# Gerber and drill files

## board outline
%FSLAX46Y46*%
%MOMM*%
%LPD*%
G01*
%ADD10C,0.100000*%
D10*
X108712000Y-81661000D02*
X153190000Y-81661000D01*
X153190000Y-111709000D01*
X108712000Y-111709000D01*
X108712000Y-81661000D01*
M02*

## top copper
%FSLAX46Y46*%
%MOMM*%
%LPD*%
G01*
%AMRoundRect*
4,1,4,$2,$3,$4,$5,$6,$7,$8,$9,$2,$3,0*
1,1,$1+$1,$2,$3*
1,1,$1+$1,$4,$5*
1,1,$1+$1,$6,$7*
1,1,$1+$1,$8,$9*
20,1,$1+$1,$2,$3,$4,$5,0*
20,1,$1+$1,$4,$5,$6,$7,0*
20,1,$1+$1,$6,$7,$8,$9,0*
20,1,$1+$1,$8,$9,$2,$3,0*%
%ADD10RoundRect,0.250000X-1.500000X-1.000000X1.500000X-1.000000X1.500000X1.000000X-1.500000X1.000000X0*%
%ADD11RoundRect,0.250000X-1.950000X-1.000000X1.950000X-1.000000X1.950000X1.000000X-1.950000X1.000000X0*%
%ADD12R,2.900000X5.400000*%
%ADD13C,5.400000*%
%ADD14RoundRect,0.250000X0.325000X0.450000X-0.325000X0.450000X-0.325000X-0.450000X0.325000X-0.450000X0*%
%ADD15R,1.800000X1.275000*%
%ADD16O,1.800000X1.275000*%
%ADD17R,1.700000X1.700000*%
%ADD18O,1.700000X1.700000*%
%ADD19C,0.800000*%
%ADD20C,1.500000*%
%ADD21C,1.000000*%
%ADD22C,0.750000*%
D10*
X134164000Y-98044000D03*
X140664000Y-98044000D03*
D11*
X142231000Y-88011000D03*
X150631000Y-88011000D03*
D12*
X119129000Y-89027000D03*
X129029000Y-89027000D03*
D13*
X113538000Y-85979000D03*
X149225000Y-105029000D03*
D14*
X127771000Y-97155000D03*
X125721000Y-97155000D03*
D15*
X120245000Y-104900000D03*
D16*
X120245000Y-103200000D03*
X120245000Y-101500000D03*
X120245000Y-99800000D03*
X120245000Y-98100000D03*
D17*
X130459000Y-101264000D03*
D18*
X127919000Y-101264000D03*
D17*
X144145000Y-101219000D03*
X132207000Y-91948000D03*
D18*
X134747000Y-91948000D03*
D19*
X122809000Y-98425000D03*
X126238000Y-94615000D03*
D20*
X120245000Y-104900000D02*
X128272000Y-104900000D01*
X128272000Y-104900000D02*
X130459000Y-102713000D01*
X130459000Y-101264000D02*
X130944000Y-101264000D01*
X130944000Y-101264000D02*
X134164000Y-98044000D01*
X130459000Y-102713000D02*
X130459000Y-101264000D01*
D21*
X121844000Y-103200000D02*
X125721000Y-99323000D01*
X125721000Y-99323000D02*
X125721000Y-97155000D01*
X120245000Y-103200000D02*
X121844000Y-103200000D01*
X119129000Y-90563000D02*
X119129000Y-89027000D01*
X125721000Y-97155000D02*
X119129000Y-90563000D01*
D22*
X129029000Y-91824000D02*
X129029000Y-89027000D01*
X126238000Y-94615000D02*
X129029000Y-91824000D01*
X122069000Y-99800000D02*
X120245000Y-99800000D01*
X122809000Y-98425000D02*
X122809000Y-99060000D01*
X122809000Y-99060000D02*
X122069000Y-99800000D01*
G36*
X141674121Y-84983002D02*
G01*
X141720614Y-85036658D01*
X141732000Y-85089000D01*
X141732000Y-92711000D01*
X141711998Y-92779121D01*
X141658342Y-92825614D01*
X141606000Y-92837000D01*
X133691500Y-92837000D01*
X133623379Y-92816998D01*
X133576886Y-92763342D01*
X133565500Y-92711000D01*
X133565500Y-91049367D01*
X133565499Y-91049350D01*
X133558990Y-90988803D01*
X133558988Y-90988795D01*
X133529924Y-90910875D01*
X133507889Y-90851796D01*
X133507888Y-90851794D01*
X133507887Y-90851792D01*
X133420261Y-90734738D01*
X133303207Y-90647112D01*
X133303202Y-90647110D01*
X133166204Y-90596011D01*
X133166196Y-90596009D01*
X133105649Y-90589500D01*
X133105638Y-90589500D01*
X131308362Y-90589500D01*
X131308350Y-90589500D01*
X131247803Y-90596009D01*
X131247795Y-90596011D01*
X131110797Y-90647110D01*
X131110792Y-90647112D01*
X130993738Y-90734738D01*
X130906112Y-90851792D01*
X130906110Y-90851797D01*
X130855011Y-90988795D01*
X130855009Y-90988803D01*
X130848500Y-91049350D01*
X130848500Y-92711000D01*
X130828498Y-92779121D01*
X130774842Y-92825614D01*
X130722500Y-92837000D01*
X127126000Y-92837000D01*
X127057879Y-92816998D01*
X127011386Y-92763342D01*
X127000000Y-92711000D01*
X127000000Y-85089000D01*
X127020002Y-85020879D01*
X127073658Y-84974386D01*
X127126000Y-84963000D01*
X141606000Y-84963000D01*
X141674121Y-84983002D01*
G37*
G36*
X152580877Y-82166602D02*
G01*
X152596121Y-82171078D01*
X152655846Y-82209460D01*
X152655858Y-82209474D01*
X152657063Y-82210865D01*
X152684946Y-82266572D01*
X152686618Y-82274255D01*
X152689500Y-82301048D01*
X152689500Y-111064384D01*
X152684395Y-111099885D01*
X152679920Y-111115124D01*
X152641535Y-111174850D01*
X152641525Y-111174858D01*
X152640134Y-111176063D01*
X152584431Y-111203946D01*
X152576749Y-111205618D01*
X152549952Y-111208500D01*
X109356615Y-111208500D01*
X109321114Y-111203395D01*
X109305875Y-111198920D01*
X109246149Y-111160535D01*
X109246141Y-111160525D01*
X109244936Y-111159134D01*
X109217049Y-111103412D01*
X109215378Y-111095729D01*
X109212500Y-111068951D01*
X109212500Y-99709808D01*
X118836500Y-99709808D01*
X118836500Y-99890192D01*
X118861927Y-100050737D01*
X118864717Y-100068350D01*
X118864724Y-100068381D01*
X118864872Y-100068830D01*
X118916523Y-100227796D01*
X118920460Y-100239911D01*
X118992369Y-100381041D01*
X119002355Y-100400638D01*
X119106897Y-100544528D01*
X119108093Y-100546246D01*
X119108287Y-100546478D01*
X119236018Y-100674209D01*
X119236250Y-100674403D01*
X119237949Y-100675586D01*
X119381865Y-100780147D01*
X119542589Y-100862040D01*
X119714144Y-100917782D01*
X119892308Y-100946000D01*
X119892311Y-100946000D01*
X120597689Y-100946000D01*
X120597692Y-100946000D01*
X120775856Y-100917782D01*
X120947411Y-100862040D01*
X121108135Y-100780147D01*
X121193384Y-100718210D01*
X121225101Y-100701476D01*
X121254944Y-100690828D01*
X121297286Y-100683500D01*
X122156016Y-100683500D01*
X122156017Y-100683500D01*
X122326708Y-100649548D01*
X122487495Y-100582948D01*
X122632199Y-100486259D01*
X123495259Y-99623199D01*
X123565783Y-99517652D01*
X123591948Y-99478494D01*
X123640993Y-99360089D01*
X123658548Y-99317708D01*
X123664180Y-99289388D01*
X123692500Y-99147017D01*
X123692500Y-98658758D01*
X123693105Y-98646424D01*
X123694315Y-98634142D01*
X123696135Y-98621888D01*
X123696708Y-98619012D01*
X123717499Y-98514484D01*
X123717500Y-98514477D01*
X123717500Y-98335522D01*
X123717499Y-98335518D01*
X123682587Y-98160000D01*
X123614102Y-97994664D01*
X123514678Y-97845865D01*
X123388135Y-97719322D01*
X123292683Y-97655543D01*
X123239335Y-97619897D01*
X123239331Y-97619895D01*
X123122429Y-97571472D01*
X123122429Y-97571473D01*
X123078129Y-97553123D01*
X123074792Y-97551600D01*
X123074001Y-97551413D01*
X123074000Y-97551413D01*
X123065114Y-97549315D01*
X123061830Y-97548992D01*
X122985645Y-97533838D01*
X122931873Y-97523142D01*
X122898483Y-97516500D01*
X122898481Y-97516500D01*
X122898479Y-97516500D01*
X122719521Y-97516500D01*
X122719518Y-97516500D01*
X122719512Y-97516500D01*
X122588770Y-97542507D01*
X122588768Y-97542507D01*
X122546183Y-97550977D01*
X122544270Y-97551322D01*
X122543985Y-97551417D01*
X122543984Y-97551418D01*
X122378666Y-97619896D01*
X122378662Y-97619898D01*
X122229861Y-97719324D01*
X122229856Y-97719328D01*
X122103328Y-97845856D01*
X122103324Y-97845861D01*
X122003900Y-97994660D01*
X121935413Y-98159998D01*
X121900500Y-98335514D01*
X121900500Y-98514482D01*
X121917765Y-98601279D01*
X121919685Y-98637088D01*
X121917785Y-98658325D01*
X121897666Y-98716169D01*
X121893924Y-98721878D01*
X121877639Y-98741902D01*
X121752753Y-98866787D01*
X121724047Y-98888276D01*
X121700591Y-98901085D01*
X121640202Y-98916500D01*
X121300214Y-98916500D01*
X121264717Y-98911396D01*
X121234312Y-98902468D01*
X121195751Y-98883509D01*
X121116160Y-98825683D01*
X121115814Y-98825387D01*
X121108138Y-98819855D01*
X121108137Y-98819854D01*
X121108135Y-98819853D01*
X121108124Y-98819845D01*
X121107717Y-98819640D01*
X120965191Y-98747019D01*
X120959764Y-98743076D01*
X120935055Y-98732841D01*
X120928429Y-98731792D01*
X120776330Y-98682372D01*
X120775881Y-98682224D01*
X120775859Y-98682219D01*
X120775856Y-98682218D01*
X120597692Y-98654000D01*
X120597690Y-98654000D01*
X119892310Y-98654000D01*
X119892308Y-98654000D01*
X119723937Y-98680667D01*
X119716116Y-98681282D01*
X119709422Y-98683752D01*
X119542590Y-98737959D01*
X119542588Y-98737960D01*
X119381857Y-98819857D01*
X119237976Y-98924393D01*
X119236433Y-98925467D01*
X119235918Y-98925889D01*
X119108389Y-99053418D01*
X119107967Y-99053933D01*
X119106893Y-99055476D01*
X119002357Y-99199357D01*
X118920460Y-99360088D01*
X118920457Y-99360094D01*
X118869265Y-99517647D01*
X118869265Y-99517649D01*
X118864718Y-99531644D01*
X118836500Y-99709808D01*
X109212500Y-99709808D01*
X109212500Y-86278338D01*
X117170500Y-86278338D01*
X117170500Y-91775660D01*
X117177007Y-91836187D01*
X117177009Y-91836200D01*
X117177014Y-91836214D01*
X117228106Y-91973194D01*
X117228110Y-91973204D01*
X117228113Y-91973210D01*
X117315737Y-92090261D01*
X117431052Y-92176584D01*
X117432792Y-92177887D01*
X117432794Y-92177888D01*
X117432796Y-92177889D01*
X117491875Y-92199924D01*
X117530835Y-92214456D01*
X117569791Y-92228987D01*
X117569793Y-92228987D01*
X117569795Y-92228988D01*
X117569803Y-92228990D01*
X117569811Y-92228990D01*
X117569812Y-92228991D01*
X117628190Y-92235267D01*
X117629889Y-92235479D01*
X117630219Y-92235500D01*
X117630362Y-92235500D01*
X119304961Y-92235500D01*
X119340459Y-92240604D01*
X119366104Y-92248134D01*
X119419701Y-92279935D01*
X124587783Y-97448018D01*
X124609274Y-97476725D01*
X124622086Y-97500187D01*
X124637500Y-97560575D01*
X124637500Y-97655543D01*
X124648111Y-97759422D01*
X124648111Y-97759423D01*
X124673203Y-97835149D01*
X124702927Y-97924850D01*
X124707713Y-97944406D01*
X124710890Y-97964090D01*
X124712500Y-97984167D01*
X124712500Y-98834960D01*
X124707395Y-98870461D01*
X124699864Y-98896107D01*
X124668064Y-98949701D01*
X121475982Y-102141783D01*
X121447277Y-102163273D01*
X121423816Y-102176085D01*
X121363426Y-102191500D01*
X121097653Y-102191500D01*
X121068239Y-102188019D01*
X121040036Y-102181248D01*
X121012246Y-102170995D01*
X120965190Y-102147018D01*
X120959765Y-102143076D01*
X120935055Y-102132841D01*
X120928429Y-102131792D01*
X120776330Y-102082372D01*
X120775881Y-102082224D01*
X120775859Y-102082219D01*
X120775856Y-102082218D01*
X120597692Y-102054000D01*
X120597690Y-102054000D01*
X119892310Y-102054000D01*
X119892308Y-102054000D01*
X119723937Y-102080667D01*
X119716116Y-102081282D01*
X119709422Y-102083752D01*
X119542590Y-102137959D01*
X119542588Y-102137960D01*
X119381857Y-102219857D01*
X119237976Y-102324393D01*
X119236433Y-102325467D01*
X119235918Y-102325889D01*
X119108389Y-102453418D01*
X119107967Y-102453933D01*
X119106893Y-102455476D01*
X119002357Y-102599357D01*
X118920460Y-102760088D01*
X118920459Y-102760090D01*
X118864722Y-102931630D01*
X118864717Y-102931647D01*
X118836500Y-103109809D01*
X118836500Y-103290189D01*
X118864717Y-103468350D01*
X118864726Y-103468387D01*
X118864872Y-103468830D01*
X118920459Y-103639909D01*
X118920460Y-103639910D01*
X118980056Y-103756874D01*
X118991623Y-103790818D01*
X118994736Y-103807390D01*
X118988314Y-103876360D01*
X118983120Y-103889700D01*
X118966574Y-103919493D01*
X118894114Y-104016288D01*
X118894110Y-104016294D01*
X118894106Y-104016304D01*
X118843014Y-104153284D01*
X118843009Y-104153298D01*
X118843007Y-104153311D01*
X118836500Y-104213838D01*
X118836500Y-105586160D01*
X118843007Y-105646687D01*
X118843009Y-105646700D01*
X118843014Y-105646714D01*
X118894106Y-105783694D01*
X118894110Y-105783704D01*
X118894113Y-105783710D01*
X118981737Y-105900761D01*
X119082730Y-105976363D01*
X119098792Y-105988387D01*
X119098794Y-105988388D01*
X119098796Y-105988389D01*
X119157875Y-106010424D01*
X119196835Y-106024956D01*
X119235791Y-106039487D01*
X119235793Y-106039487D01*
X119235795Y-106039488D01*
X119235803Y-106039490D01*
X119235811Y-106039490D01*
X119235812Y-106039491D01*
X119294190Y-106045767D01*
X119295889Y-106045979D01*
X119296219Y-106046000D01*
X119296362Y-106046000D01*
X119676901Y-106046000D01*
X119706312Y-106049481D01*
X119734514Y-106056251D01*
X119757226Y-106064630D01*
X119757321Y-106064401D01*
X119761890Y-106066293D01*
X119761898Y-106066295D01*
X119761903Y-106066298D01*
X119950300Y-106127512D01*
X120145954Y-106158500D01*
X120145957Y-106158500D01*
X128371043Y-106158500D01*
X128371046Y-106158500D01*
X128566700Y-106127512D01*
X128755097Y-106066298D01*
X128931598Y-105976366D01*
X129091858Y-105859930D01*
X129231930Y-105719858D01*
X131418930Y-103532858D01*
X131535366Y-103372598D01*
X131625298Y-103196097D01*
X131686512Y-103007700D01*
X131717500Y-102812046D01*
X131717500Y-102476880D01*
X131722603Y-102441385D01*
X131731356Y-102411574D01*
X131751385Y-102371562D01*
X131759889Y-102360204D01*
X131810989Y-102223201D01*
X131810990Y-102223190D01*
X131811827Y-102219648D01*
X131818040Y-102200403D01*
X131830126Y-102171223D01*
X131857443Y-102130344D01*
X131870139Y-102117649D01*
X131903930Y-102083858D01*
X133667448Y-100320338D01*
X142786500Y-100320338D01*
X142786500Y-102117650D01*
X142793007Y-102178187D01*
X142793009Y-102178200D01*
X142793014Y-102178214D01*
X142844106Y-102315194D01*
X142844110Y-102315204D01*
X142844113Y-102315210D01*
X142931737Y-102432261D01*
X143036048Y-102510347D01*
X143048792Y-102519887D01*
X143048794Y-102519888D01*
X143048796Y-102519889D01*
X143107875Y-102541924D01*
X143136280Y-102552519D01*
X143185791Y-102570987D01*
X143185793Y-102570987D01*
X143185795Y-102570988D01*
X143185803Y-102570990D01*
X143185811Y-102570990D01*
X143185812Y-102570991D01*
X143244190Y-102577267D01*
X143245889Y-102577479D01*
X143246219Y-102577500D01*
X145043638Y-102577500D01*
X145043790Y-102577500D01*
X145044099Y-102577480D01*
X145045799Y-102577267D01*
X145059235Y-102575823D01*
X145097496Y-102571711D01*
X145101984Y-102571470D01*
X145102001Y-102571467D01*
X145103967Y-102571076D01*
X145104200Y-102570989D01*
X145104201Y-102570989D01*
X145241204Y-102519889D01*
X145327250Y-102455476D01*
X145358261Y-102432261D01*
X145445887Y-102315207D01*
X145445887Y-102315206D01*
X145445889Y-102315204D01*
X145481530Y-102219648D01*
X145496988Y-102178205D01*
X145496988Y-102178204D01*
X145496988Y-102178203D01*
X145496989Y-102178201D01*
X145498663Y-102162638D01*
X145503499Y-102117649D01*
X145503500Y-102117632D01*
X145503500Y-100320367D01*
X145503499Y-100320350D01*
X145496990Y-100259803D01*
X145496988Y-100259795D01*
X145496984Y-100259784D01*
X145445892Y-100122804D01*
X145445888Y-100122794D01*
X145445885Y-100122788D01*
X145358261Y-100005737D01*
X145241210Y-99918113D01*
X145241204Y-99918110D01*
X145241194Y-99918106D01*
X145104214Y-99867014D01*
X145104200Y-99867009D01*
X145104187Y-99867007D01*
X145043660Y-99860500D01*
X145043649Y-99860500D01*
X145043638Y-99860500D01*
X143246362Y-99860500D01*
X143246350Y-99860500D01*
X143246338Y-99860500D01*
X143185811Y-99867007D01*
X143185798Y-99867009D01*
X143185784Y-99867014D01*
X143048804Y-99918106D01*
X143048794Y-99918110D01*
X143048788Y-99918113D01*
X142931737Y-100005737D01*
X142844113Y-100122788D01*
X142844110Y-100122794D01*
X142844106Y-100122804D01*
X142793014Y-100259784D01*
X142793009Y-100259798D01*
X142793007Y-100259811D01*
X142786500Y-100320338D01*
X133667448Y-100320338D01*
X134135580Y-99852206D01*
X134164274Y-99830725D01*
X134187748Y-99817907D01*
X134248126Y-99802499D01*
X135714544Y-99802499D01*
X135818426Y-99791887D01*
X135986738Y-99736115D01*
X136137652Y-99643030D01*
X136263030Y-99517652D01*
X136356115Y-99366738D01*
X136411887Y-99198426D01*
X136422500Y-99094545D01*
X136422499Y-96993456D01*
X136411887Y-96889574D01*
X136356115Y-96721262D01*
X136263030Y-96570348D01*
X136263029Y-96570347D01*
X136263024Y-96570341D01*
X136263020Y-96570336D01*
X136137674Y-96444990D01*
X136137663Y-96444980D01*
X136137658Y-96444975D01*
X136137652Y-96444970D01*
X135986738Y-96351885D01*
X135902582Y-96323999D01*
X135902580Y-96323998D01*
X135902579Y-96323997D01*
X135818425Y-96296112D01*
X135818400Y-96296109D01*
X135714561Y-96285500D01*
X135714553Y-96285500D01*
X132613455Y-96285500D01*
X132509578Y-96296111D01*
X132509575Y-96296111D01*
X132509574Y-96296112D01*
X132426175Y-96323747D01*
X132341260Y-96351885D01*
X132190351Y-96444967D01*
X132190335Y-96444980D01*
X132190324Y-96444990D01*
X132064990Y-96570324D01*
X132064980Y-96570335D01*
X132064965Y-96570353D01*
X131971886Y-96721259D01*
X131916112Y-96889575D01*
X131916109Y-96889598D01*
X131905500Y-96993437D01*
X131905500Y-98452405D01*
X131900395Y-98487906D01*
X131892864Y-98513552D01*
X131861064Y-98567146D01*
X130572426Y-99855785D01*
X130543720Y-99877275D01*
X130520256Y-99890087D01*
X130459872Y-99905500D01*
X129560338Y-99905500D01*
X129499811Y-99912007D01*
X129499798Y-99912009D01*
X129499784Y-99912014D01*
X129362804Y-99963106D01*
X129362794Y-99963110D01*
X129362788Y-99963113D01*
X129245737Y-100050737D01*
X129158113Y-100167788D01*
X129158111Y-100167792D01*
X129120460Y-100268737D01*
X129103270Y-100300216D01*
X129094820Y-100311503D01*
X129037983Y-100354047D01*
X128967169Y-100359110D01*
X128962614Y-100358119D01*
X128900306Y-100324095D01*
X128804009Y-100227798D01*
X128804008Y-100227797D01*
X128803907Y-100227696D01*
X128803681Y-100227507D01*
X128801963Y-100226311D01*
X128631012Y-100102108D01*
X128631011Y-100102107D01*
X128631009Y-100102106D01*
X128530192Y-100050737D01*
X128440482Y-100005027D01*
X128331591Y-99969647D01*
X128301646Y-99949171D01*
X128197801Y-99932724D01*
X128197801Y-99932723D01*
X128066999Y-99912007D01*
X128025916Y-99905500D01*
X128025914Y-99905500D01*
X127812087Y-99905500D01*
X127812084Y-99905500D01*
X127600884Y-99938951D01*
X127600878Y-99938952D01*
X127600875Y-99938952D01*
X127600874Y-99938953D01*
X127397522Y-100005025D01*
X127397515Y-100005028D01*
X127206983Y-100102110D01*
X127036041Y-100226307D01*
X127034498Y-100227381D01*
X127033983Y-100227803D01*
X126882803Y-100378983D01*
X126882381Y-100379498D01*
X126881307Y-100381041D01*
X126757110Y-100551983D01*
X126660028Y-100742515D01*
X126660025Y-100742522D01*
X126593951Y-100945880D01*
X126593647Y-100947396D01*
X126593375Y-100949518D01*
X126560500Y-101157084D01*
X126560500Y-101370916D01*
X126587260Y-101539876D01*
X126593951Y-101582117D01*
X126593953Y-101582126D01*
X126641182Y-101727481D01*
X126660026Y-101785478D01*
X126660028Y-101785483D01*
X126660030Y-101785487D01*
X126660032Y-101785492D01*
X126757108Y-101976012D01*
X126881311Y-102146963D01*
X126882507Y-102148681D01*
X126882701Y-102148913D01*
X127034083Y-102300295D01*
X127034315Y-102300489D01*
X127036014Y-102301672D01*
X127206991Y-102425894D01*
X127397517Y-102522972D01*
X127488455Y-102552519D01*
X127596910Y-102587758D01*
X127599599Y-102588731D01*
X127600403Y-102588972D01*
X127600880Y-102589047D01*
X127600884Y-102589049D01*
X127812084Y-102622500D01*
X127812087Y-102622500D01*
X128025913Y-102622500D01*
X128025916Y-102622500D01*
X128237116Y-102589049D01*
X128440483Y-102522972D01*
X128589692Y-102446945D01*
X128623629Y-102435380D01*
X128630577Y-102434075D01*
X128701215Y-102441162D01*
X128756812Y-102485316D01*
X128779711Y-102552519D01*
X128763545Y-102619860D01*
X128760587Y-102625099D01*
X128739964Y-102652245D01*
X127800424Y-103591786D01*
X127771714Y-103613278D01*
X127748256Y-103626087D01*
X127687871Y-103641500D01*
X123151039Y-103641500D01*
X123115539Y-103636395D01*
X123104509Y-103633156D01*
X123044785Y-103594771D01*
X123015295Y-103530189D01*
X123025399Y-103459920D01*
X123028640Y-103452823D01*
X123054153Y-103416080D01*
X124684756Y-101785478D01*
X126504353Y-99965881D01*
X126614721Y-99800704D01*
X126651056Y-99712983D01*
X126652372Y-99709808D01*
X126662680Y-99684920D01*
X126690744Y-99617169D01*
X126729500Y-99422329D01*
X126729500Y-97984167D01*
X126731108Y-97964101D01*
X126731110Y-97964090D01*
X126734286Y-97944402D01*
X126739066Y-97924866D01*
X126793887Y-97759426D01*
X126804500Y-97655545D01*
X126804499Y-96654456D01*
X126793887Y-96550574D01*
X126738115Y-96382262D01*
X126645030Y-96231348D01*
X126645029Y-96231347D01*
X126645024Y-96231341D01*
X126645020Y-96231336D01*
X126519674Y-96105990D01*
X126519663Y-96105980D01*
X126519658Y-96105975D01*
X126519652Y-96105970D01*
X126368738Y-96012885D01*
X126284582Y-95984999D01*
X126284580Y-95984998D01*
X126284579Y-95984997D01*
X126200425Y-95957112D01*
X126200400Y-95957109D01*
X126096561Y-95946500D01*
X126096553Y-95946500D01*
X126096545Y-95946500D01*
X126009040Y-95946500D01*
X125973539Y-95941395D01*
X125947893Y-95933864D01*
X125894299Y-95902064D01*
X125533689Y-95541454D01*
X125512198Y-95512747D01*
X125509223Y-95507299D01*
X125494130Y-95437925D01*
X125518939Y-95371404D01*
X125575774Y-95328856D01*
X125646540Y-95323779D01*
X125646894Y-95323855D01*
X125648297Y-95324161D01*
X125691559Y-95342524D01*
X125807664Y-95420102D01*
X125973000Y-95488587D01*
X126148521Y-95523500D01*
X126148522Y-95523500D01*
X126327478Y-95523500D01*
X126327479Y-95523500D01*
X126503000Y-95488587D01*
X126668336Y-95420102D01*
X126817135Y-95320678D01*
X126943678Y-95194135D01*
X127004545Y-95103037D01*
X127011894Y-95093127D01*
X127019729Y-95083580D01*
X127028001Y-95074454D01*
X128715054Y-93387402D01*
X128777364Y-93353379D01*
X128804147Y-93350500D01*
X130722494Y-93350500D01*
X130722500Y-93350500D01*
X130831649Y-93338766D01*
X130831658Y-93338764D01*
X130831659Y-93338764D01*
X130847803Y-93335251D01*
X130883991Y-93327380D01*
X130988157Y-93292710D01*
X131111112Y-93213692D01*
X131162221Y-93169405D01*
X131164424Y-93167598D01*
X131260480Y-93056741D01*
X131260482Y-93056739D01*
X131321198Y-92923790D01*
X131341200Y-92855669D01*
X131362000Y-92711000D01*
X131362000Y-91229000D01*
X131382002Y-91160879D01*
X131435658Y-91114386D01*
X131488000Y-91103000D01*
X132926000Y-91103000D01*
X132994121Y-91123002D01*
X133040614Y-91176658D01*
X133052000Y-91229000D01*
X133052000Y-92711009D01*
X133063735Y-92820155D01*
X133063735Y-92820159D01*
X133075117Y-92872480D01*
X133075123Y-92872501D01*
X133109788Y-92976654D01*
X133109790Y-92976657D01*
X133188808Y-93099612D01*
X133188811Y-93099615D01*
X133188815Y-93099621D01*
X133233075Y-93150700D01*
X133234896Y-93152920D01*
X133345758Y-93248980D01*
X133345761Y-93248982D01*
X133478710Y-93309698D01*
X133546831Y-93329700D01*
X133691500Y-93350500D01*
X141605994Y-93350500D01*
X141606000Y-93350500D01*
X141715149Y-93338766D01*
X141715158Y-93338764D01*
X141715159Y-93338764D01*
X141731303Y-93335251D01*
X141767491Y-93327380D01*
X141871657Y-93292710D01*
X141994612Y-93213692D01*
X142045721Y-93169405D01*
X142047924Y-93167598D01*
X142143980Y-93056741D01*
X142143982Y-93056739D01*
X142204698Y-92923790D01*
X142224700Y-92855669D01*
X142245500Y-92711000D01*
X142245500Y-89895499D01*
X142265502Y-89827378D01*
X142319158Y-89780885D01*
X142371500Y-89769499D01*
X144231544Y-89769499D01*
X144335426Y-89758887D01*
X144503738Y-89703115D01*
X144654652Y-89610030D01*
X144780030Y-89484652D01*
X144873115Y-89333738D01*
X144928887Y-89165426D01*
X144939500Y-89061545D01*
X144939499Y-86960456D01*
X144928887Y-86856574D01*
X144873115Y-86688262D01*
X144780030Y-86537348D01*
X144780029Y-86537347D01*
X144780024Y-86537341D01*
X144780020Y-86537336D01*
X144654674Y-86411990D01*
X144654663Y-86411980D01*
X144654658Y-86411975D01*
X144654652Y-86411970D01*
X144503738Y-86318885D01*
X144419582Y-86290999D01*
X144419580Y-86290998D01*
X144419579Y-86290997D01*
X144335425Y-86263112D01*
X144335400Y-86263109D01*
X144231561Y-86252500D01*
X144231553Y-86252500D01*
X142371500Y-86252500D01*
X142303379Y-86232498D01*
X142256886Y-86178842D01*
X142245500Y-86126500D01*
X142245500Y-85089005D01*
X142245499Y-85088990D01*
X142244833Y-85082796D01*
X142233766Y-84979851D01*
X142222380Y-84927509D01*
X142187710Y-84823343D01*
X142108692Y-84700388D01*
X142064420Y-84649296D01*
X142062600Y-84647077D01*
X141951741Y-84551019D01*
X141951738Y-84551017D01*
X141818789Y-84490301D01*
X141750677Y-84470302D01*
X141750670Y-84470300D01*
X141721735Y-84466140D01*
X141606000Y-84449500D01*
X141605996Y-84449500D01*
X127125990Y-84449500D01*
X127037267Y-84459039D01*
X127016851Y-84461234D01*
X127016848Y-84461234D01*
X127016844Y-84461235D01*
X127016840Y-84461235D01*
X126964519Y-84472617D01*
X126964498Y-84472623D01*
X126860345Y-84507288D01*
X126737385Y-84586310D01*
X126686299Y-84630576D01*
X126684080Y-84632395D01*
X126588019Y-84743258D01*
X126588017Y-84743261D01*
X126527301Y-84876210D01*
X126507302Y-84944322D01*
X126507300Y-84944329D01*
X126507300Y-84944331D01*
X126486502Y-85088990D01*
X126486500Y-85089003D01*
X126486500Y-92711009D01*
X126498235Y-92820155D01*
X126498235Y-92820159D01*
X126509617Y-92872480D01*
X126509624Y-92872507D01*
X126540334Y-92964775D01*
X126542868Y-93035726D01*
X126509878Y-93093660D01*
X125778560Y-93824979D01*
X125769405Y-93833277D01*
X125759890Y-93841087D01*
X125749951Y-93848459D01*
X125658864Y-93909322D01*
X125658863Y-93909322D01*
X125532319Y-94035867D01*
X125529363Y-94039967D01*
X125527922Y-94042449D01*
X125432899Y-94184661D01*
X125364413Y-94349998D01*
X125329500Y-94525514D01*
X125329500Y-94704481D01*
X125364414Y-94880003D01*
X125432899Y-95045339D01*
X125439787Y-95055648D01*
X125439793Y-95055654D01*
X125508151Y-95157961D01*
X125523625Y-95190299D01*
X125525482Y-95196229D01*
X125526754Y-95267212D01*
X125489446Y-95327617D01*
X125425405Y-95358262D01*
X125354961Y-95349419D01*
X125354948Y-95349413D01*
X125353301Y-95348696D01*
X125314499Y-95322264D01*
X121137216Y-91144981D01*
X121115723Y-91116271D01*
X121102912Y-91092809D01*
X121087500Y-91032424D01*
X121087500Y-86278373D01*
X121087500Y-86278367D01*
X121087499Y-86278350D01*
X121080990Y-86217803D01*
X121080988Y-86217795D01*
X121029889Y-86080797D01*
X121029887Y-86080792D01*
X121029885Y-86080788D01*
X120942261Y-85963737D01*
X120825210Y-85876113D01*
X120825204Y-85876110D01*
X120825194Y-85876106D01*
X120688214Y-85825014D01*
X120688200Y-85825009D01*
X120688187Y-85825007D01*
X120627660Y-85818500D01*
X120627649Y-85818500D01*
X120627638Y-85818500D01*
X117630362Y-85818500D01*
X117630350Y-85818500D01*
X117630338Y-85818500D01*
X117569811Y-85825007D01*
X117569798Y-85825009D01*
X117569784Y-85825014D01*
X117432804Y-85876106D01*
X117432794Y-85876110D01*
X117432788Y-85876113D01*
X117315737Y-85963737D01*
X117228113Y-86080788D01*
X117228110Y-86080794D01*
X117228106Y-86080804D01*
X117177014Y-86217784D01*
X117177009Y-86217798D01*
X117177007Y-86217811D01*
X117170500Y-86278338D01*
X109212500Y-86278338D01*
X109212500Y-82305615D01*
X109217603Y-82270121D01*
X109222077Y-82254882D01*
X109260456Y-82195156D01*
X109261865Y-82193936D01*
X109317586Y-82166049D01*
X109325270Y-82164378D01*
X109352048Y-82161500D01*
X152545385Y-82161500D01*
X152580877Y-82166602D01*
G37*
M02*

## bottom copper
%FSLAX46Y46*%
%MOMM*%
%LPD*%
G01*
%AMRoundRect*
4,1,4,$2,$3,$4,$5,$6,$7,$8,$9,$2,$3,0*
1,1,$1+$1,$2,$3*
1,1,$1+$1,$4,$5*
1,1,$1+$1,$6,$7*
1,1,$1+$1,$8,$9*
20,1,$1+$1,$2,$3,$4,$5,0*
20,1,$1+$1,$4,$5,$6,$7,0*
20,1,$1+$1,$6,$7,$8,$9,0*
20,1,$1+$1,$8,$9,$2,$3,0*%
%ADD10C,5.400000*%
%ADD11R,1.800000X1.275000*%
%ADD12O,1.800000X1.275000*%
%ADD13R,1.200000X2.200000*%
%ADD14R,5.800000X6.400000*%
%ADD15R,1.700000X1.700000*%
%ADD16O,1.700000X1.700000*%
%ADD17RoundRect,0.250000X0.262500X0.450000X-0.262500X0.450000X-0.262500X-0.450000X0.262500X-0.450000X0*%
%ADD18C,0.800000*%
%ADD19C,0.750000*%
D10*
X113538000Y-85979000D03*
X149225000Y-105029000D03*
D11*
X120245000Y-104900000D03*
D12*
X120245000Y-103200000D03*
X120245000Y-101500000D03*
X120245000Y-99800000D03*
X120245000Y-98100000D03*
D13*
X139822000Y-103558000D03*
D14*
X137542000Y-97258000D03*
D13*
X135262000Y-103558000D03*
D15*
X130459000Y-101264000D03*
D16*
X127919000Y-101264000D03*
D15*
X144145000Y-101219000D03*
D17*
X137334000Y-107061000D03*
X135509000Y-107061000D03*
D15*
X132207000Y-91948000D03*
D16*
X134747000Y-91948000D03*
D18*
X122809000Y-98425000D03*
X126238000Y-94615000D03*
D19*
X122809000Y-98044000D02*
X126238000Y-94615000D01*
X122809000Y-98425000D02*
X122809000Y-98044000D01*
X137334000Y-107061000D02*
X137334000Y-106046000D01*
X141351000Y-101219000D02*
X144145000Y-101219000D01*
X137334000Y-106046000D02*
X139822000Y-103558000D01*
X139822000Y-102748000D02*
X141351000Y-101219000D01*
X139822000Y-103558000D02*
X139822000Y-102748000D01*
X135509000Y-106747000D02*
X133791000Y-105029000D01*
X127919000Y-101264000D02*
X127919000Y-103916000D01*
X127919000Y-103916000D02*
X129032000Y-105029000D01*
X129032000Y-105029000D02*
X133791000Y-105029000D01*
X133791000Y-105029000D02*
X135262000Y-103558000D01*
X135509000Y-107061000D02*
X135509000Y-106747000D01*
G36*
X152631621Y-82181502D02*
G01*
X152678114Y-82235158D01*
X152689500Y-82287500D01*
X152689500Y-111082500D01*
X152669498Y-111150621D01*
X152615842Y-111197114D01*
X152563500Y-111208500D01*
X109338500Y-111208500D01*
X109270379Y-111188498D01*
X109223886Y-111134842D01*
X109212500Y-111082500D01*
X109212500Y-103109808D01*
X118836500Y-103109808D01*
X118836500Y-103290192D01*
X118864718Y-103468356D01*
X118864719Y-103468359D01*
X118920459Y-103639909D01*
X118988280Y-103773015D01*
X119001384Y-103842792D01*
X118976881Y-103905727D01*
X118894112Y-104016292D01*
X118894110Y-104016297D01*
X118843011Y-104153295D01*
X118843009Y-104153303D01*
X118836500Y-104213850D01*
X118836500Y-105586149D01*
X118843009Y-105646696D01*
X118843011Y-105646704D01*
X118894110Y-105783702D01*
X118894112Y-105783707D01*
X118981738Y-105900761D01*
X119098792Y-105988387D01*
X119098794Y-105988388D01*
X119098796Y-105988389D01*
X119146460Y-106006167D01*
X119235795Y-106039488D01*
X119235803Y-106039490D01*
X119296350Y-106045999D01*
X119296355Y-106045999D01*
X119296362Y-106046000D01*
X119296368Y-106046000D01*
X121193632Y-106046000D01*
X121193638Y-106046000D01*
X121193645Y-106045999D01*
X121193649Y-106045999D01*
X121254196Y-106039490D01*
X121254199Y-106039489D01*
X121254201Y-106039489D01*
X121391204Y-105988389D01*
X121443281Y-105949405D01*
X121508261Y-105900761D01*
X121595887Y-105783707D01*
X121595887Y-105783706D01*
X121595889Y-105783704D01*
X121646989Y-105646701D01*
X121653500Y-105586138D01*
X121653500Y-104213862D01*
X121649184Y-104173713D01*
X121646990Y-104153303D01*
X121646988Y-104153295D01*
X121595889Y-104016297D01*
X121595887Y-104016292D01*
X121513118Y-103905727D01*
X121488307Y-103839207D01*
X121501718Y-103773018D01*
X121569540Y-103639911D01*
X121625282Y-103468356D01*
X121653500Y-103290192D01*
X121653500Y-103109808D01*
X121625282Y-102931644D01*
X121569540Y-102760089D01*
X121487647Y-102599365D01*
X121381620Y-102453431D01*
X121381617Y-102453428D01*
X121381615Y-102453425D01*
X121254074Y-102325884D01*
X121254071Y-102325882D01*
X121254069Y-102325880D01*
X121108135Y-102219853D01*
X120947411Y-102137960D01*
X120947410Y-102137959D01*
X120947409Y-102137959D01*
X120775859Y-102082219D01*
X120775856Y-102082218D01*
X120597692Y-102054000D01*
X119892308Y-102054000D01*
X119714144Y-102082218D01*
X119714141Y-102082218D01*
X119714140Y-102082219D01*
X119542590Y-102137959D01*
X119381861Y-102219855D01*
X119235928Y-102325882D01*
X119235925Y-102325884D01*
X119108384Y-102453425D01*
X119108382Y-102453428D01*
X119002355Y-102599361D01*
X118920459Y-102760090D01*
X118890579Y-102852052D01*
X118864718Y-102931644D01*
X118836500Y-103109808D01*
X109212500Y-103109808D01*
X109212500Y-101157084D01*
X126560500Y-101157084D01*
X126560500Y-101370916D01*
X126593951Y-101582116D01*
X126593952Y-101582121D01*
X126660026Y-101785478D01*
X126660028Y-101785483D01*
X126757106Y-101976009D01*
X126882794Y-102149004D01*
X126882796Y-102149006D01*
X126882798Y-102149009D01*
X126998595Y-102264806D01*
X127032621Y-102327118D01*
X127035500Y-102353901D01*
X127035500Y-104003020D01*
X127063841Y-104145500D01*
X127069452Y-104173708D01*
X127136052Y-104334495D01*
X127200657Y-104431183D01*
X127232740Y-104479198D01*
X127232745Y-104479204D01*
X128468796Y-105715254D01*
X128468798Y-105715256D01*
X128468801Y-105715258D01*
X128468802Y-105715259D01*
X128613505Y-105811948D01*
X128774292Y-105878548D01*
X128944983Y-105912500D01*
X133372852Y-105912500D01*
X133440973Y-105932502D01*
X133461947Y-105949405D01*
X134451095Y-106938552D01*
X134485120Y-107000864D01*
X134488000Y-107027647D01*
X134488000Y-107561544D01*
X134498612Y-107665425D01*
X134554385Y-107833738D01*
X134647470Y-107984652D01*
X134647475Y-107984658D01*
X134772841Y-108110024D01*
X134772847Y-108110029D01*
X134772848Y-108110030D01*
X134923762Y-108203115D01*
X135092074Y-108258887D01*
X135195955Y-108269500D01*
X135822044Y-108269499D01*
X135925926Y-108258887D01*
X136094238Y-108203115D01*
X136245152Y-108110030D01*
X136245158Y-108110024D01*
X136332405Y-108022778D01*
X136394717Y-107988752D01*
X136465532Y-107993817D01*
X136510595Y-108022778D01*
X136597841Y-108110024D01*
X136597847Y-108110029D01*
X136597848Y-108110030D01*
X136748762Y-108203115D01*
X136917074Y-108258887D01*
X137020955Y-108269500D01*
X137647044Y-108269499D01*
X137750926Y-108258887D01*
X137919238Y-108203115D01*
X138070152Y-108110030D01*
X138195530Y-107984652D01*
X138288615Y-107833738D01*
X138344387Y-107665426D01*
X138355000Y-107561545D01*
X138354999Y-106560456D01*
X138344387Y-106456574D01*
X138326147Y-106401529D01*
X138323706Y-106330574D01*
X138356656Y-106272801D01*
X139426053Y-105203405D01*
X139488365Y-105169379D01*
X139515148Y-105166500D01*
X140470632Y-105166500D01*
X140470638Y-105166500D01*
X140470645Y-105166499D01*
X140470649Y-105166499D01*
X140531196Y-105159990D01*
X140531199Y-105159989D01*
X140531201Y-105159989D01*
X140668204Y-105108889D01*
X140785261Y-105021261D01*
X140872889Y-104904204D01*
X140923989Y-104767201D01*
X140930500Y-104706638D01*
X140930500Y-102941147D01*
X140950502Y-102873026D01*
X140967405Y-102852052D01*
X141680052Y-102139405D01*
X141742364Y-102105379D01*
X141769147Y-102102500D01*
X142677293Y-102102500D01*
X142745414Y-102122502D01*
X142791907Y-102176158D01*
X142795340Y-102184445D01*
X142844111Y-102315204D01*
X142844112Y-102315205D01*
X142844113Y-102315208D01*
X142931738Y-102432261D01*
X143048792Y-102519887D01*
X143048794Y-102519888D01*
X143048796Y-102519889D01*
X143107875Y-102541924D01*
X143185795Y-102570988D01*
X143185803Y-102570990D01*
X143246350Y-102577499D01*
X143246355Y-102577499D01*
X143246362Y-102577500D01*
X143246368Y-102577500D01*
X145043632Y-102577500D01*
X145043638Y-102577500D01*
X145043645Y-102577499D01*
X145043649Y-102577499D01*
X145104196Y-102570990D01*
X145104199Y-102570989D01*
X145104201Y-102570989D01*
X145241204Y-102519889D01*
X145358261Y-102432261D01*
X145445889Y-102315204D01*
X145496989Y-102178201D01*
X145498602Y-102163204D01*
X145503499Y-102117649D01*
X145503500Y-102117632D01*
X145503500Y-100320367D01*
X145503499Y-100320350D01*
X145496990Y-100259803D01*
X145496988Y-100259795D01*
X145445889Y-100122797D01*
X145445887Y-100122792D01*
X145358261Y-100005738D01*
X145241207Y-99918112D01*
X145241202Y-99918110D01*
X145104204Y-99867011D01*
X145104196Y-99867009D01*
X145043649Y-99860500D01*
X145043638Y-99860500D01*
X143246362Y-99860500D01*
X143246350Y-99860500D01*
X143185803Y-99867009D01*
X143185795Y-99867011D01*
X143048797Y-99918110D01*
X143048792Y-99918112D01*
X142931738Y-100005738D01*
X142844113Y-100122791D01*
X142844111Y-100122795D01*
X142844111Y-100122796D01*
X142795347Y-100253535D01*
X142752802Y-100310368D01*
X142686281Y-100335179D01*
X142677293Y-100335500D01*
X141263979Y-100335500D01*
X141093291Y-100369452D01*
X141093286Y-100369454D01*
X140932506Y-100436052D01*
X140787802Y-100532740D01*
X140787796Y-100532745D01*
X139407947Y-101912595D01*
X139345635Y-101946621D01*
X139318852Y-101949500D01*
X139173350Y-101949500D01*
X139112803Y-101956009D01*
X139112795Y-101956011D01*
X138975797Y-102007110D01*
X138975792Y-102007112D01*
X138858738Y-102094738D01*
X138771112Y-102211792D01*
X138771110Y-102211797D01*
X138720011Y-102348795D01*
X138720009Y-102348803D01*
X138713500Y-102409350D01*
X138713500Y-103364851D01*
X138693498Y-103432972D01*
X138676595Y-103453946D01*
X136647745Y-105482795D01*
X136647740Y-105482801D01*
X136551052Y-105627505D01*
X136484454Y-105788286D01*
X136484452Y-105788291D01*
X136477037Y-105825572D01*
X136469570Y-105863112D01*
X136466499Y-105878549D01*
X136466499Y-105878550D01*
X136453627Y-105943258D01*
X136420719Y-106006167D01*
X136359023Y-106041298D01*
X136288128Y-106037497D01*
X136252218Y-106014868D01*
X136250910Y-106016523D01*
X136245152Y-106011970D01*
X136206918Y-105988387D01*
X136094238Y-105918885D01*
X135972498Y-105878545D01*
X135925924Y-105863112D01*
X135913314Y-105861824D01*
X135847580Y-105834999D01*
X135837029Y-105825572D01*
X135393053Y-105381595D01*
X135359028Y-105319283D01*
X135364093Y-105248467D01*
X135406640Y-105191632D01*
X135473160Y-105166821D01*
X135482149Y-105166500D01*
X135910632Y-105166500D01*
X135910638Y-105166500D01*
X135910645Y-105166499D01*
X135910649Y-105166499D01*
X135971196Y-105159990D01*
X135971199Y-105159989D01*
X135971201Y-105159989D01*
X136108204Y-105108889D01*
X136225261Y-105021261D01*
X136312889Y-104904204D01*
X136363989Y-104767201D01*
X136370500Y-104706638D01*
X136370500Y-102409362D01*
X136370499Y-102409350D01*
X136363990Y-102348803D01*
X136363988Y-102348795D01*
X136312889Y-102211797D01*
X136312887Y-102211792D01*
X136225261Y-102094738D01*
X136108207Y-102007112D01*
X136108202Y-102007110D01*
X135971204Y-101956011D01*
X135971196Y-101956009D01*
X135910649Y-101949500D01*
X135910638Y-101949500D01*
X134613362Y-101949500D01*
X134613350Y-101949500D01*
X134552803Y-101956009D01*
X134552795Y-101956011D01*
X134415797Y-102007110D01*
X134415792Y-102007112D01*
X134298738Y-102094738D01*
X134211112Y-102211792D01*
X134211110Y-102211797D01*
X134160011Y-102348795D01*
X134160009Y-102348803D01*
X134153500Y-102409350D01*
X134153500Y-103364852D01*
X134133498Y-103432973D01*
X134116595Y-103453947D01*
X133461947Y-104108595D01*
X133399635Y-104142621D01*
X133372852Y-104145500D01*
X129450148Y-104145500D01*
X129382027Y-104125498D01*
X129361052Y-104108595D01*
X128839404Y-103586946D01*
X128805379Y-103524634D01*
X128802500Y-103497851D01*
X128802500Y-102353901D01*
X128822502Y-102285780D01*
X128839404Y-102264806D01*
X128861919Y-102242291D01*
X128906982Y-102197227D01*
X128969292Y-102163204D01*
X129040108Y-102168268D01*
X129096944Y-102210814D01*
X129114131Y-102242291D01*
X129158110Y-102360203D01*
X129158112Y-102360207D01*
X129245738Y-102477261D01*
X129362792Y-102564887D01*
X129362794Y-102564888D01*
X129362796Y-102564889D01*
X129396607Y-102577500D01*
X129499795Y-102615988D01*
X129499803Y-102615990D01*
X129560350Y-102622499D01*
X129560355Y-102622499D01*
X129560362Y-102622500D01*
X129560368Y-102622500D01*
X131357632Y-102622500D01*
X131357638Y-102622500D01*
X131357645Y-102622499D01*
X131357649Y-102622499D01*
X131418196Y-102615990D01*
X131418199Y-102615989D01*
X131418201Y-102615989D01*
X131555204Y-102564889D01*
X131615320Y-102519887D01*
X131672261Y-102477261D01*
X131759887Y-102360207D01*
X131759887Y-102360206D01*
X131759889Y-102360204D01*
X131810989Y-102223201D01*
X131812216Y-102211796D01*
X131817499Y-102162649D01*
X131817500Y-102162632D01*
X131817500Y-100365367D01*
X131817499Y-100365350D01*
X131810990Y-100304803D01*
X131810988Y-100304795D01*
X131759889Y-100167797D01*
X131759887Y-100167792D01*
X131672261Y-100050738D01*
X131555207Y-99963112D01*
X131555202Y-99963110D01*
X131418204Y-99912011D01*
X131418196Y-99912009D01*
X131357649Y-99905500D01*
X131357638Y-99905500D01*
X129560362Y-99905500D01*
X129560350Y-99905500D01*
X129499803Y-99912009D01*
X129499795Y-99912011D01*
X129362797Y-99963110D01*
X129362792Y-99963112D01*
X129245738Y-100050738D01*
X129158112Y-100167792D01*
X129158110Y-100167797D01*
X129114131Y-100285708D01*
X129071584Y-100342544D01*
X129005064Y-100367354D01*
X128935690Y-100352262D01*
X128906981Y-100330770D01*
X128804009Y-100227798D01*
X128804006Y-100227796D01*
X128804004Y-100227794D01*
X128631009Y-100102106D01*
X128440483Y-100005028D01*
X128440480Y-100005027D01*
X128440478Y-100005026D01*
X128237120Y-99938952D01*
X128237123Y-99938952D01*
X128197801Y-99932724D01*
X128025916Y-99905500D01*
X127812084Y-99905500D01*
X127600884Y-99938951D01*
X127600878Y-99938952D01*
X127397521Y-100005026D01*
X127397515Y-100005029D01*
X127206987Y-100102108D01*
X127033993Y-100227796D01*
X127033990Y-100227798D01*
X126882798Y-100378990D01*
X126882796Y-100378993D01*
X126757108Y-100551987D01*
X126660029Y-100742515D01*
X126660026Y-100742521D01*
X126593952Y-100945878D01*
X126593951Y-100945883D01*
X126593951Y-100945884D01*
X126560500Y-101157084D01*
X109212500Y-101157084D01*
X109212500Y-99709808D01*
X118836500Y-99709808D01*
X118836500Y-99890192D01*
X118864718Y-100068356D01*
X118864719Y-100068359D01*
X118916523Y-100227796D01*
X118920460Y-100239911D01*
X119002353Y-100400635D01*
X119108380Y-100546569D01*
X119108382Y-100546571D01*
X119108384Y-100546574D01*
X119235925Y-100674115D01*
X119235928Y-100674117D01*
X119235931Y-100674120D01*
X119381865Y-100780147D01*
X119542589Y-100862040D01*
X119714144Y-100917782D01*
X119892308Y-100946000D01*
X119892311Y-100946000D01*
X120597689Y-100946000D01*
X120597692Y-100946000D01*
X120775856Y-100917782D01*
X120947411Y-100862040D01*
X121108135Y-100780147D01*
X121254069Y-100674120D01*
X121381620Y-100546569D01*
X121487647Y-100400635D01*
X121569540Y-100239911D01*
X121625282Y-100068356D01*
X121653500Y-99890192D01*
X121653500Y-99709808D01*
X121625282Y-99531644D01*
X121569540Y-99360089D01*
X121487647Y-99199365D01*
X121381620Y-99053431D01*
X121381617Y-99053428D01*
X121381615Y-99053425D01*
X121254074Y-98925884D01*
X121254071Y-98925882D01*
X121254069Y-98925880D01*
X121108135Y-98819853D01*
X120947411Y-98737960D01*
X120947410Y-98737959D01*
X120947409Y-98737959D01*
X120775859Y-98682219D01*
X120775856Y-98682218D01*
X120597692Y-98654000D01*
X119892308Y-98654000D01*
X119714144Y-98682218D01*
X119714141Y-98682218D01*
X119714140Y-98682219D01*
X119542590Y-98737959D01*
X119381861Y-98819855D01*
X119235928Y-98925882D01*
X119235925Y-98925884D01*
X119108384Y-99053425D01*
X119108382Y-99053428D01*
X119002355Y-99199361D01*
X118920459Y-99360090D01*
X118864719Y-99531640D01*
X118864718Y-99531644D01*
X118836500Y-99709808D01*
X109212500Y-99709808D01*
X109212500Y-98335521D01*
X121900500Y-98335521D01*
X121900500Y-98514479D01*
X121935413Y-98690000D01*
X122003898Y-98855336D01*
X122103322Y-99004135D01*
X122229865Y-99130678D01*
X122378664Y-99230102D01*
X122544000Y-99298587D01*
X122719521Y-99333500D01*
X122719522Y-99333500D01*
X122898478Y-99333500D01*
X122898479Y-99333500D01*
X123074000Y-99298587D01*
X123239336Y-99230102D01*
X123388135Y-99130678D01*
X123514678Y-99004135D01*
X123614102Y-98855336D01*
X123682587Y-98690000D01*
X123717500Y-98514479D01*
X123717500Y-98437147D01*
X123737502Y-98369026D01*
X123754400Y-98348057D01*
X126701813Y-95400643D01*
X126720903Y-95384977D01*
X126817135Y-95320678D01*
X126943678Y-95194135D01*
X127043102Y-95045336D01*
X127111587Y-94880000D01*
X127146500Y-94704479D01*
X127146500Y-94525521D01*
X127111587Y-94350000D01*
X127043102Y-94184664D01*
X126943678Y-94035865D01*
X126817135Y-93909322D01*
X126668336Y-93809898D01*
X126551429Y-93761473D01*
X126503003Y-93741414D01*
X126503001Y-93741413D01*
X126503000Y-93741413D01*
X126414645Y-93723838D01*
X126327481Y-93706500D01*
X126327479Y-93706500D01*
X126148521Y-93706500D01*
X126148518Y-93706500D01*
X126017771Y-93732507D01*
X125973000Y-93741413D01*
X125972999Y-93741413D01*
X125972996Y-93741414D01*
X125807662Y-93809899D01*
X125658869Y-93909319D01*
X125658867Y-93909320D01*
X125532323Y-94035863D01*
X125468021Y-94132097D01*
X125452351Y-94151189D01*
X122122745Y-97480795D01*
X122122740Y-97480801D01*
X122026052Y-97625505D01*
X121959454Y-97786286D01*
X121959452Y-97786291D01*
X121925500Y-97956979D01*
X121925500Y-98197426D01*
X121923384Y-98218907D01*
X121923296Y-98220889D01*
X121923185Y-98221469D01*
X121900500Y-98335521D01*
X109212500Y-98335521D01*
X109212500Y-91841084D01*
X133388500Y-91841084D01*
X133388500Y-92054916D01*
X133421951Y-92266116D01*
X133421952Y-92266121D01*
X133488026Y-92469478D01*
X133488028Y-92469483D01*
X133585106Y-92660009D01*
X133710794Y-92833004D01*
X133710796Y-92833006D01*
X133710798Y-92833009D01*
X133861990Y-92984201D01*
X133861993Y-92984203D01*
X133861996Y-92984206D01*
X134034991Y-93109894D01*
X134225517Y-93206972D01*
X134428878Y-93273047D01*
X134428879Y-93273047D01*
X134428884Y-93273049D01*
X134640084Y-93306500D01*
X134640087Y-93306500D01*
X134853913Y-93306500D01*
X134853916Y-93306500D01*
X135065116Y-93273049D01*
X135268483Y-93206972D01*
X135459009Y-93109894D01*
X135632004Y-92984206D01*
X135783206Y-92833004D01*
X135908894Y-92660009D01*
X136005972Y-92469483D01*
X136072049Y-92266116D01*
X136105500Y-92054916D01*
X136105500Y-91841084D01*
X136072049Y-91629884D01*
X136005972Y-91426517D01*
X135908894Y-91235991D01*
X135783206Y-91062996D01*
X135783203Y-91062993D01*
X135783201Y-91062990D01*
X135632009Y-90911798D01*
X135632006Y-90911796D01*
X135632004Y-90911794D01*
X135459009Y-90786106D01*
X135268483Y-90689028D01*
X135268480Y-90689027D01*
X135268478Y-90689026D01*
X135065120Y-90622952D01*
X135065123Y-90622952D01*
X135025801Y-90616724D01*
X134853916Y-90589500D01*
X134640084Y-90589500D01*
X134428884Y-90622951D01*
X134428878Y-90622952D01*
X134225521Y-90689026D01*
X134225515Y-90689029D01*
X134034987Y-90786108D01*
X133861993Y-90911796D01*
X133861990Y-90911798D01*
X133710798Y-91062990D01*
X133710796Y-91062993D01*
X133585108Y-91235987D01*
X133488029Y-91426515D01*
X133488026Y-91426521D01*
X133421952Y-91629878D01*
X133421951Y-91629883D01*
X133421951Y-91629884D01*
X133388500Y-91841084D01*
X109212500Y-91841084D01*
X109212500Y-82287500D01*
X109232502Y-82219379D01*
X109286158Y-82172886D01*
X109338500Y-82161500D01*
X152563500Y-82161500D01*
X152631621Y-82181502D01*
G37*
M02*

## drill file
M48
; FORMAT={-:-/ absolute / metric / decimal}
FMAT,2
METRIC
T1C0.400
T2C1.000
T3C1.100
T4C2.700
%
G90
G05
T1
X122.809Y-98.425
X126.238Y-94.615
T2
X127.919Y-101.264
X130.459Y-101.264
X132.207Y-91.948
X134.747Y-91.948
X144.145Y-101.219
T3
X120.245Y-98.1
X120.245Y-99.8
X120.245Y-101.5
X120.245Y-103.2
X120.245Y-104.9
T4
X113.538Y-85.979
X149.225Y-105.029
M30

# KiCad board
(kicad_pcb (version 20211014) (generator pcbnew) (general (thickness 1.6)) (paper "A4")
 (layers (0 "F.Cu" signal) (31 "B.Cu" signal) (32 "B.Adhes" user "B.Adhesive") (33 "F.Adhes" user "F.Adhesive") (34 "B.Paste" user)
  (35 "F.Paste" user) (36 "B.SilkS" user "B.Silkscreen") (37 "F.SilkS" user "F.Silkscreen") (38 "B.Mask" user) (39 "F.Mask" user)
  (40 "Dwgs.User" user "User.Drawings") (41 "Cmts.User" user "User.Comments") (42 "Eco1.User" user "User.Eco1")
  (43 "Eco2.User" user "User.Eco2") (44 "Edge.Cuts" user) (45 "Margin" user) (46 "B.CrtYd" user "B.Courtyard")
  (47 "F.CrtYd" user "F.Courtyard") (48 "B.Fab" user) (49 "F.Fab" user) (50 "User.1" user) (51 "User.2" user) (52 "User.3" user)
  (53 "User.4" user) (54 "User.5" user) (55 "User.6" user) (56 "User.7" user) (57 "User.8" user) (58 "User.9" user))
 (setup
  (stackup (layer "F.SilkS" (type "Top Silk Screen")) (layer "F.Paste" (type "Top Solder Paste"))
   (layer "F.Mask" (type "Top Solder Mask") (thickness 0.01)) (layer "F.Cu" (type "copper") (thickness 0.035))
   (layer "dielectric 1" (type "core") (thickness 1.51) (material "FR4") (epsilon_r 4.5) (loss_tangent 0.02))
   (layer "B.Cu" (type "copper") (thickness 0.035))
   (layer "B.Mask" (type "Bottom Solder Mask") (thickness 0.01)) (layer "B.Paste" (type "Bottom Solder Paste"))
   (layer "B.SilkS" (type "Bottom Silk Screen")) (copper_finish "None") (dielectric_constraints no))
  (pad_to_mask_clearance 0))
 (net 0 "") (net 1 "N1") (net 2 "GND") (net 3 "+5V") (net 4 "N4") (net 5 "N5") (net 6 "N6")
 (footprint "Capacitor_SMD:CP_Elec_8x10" (layer "F.Cu") (at 137.414 98.044)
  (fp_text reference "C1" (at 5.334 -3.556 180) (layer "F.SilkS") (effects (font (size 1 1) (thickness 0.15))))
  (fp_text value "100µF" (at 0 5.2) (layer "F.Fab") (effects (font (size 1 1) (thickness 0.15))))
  (pad "1" smd roundrect (at -3.25 0) (size 3.5 2.5) (layers "F.Cu" "F.Paste" "F.Mask") (roundrect_rratio 0.1) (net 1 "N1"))
  (pad "2" smd roundrect (at 3.25 0) (size 3.5 2.5) (layers "F.Cu" "F.Paste" "F.Mask") (roundrect_rratio 0.1) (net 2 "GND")))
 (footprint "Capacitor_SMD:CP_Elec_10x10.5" (layer "F.Cu") (at 146.431 88.011)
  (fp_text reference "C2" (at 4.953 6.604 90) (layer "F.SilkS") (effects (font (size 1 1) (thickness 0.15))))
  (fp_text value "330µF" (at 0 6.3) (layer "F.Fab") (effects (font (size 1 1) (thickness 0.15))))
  (pad "1" smd roundrect (at -4.2 0) (size 4.4 2.5) (layers "F.Cu" "F.Paste" "F.Mask") (roundrect_rratio 0.1) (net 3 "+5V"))
  (pad "2" smd roundrect (at 4.2 0) (size 4.4 2.5) (layers "F.Cu" "F.Paste" "F.Mask") (roundrect_rratio 0.1) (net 2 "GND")))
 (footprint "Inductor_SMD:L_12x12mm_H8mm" (layer "F.Cu") (at 124.079 89.027)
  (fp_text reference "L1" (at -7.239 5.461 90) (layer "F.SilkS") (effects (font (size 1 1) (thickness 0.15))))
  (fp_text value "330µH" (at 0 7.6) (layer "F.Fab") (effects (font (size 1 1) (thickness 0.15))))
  (pad "1" smd rect (at -4.95 0) (size 2.9 5.4) (layers "F.Cu" "F.Paste" "F.Mask") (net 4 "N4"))
  (pad "2" smd rect (at 4.95 0) (size 2.9 5.4) (layers "F.Cu" "F.Paste" "F.Mask") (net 3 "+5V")))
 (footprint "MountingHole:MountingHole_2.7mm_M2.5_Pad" (layer "F.Cu") (at 113.538 85.979)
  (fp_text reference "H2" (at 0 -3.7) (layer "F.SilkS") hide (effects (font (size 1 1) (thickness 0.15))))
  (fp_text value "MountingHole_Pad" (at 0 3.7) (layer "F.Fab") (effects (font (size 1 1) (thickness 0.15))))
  (pad "1" thru_hole circle (at 0 0) (size 5.4 5.4) (drill 2.7) (layers *.Cu *.Mask) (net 2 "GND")))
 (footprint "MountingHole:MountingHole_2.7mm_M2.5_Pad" (layer "F.Cu") (at 149.225 105.029 90)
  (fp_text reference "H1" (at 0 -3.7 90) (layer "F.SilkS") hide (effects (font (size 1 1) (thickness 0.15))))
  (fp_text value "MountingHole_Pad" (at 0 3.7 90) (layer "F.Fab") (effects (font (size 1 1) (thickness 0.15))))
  (pad "1" thru_hole circle (at 0 0 90) (size 5.4 5.4) (drill 2.7) (layers *.Cu *.Mask) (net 2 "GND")))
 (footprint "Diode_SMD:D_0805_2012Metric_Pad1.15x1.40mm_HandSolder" (layer "F.Cu") (at 126.746 97.155 180)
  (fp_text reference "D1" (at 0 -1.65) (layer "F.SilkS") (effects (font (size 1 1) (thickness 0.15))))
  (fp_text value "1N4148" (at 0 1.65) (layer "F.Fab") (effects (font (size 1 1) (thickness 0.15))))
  (pad "1" smd roundrect (at -1.025 0 180) (size 1.15 1.4) (layers "F.Cu" "F.Paste" "F.Mask") (roundrect_rratio 0.2173913043) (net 2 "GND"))
  (pad "2" smd roundrect (at 1.025 0 180) (size 1.15 1.4) (layers "F.Cu" "F.Paste" "F.Mask") (roundrect_rratio 0.2173913043) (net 4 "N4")))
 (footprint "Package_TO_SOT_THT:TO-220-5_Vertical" (layer "F.Cu") (at 120.245 104.9 90)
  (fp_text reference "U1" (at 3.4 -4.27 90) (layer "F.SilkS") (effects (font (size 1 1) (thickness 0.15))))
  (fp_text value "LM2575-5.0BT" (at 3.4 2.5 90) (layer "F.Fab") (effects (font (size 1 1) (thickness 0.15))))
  (pad "1" thru_hole rect (at 0 0 90) (size 1.275 1.8) (drill 1.1) (layers *.Cu *.Mask) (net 1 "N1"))
  (pad "2" thru_hole oval (at 1.7 0 90) (size 1.275 1.8) (drill 1.1) (layers *.Cu *.Mask) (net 4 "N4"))
  (pad "3" thru_hole oval (at 3.4 0 90) (size 1.275 1.8) (drill 1.1) (layers *.Cu *.Mask) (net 2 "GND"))
  (pad "4" thru_hole oval (at 5.1 0 90) (size 1.275 1.8) (drill 1.1) (layers *.Cu *.Mask) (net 3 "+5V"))
  (pad "5" thru_hole oval (at 6.8 0 90) (size 1.275 1.8) (drill 1.1) (layers *.Cu *.Mask) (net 2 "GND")))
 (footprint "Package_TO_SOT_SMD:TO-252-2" (layer "B.Cu") (at 137.542 99.358 90)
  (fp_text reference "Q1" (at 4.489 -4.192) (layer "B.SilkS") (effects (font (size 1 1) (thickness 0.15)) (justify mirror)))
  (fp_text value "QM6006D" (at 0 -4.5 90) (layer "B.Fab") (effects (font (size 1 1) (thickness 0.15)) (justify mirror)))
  (pad "" smd rect (at 0.425 -1.525 90) (size 3.05 2.75) (layers "B.Paste"))
  (pad "" smd rect (at 3.775 -1.525 90) (size 3.05 2.75) (layers "B.Paste"))
  (pad "" smd rect (at 0.425 1.525 90) (size 3.05 2.75) (layers "B.Paste"))
  (pad "" smd rect (at 3.775 1.525 90) (size 3.05 2.75) (layers "B.Paste"))
  (pad "1" smd rect (at -4.2 2.28 90) (size 2.2 1.2) (layers "B.Cu" "B.Paste" "B.Mask") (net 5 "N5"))
  (pad "2" smd rect (at 2.1 0 90) (size 6.4 5.8) (layers "B.Cu" "B.Mask") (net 2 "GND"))
  (pad "3" smd rect (at -4.2 -2.28 90) (size 2.2 1.2) (layers "B.Cu" "B.Paste" "B.Mask") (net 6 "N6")))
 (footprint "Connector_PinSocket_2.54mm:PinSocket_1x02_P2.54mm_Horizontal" (layer "B.Cu") (at 130.459 101.264 90)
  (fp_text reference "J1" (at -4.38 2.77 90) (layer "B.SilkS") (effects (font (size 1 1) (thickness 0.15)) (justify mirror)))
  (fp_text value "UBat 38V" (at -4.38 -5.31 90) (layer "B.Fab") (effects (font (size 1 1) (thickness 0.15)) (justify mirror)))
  (pad "1" thru_hole rect (at 0 0 90) (size 1.7 1.7) (drill 1) (layers *.Cu *.Mask) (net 1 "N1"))
  (pad "2" thru_hole oval (at 0 -2.54 90) (size 1.7 1.7) (drill 1) (layers *.Cu *.Mask) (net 6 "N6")))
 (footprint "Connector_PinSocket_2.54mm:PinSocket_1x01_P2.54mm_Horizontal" (layer "B.Cu") (at 144.145 101.219 90)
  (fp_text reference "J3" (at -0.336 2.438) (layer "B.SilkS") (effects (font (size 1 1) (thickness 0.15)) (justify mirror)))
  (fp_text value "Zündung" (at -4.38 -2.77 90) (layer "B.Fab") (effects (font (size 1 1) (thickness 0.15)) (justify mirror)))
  (pad "1" thru_hole rect (at 0 0 90) (size 1.7 1.7) (drill 1) (layers *.Cu *.Mask) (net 5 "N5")))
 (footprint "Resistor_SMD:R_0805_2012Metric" (layer "B.Cu") (at 136.4215 107.061 180)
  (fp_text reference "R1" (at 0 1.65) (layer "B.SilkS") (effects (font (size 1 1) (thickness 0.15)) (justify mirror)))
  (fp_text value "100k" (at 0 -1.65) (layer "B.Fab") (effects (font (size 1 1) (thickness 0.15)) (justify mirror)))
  (pad "1" smd roundrect (at -0.9125 0 180) (size 1.025 1.4) (layers "B.Cu" "B.Paste" "B.Mask") (roundrect_rratio 0.243902439) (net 5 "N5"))
  (pad "2" smd roundrect (at 0.9125 0 180) (size 1.025 1.4) (layers "B.Cu" "B.Paste" "B.Mask") (roundrect_rratio 0.243902439) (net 6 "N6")))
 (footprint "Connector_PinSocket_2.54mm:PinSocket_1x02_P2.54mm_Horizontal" (layer "B.Cu") (at 132.207 91.948 -90)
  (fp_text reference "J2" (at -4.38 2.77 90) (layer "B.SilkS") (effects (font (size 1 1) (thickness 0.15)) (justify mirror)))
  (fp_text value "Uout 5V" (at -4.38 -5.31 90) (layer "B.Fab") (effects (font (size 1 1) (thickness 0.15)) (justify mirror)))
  (pad "1" thru_hole rect (at 0 0 270) (size 1.7 1.7) (drill 1) (layers *.Cu *.Mask) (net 2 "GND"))
  (pad "2" thru_hole oval (at 0 -2.54 270) (size 1.7 1.7) (drill 1) (layers *.Cu *.Mask) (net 3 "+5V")))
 (gr_rect (start 108.712 81.661) (end 153.19 111.709) (layer "Edge.Cuts") (width 0.1) (fill none))
 (segment (start 120.245 104.9) (end 128.272 104.9) (width 1.5) (layer "F.Cu") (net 1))
 (segment (start 128.272 104.9) (end 130.459 102.713) (width 1.5) (layer "F.Cu") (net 1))
 (segment (start 130.459 101.264) (end 130.944 101.264) (width 1.5) (layer "F.Cu") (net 1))
 (segment (start 130.944 101.264) (end 134.164 98.044) (width 1.5) (layer "F.Cu") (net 1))
 (segment (start 130.459 102.713) (end 130.459 101.264) (width 1.5) (layer "F.Cu") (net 1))
 (segment (start 121.844 103.2) (end 125.721 99.323) (width 1) (layer "F.Cu") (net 4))
 (segment (start 125.721 99.323) (end 125.721 97.155) (width 1) (layer "F.Cu") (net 4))
 (segment (start 120.245 103.2) (end 121.844 103.2) (width 1) (layer "F.Cu") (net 4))
 (segment (start 119.129 90.563) (end 119.129 89.027) (width 1) (layer "F.Cu") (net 4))
 (segment (start 125.721 97.155) (end 119.129 90.563) (width 1) (layer "F.Cu") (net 4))
 (segment (start 129.029 91.824) (end 129.029 89.027) (width 0.75) (layer "F.Cu") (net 3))
 (segment (start 126.238 94.615) (end 129.029 91.824) (width 0.75) (layer "F.Cu") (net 3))
 (segment (start 122.069 99.8) (end 120.245 99.8) (width 0.75) (layer "F.Cu") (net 3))
 (segment (start 122.809 98.425) (end 122.809 99.06) (width 0.75) (layer "F.Cu") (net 3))
 (segment (start 122.809 99.06) (end 122.069 99.8) (width 0.75) (layer "F.Cu") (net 3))
 (via (at 122.809 98.425) (size 0.8) (drill 0.4) (layers "F.Cu" "B.Cu") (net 3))
 (via (at 126.238 94.615) (size 0.8) (drill 0.4) (layers "F.Cu" "B.Cu") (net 3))
 (segment (start 122.809 98.044) (end 126.238 94.615) (width 0.75) (layer "B.Cu") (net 3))
 (segment (start 122.809 98.425) (end 122.809 98.044) (width 0.75) (layer "B.Cu") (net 3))
 (segment (start 137.334 107.061) (end 137.334 106.046) (width 0.75) (layer "B.Cu") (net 5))
 (segment (start 141.351 101.219) (end 144.145 101.219) (width 0.75) (layer "B.Cu") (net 5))
 (segment (start 137.334 106.046) (end 139.822 103.558) (width 0.75) (layer "B.Cu") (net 5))
 (segment (start 139.822 102.748) (end 141.351 101.219) (width 0.75) (layer "B.Cu") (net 5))
 (segment (start 139.822 103.558) (end 139.822 102.748) (width 0.75) (layer "B.Cu") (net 5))
 (segment (start 135.509 106.747) (end 133.791 105.029) (width 0.75) (layer "B.Cu") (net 6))
 (segment (start 127.919 101.264) (end 127.919 103.916) (width 0.75) (layer "B.Cu") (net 6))
 (segment (start 127.919 103.916) (end 129.032 105.029) (width 0.75) (layer "B.Cu") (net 6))
 (segment (start 129.032 105.029) (end 133.791 105.029) (width 0.75) (layer "B.Cu") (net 6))
 (segment (start 133.791 105.029) (end 135.262 103.558) (width 0.75) (layer "B.Cu") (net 6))
 (segment (start 135.509 107.061) (end 135.509 106.747) (width 0.75) (layer "B.Cu") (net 6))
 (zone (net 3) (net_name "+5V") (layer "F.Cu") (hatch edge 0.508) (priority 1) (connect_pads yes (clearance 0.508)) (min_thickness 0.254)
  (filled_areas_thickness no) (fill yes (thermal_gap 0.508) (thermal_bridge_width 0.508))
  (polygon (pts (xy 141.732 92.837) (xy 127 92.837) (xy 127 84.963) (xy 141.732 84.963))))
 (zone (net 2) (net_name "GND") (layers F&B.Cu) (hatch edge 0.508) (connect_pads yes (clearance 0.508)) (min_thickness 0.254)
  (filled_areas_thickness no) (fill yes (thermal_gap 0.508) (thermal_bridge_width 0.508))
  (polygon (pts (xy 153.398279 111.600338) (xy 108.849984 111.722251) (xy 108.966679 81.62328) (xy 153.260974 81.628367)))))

